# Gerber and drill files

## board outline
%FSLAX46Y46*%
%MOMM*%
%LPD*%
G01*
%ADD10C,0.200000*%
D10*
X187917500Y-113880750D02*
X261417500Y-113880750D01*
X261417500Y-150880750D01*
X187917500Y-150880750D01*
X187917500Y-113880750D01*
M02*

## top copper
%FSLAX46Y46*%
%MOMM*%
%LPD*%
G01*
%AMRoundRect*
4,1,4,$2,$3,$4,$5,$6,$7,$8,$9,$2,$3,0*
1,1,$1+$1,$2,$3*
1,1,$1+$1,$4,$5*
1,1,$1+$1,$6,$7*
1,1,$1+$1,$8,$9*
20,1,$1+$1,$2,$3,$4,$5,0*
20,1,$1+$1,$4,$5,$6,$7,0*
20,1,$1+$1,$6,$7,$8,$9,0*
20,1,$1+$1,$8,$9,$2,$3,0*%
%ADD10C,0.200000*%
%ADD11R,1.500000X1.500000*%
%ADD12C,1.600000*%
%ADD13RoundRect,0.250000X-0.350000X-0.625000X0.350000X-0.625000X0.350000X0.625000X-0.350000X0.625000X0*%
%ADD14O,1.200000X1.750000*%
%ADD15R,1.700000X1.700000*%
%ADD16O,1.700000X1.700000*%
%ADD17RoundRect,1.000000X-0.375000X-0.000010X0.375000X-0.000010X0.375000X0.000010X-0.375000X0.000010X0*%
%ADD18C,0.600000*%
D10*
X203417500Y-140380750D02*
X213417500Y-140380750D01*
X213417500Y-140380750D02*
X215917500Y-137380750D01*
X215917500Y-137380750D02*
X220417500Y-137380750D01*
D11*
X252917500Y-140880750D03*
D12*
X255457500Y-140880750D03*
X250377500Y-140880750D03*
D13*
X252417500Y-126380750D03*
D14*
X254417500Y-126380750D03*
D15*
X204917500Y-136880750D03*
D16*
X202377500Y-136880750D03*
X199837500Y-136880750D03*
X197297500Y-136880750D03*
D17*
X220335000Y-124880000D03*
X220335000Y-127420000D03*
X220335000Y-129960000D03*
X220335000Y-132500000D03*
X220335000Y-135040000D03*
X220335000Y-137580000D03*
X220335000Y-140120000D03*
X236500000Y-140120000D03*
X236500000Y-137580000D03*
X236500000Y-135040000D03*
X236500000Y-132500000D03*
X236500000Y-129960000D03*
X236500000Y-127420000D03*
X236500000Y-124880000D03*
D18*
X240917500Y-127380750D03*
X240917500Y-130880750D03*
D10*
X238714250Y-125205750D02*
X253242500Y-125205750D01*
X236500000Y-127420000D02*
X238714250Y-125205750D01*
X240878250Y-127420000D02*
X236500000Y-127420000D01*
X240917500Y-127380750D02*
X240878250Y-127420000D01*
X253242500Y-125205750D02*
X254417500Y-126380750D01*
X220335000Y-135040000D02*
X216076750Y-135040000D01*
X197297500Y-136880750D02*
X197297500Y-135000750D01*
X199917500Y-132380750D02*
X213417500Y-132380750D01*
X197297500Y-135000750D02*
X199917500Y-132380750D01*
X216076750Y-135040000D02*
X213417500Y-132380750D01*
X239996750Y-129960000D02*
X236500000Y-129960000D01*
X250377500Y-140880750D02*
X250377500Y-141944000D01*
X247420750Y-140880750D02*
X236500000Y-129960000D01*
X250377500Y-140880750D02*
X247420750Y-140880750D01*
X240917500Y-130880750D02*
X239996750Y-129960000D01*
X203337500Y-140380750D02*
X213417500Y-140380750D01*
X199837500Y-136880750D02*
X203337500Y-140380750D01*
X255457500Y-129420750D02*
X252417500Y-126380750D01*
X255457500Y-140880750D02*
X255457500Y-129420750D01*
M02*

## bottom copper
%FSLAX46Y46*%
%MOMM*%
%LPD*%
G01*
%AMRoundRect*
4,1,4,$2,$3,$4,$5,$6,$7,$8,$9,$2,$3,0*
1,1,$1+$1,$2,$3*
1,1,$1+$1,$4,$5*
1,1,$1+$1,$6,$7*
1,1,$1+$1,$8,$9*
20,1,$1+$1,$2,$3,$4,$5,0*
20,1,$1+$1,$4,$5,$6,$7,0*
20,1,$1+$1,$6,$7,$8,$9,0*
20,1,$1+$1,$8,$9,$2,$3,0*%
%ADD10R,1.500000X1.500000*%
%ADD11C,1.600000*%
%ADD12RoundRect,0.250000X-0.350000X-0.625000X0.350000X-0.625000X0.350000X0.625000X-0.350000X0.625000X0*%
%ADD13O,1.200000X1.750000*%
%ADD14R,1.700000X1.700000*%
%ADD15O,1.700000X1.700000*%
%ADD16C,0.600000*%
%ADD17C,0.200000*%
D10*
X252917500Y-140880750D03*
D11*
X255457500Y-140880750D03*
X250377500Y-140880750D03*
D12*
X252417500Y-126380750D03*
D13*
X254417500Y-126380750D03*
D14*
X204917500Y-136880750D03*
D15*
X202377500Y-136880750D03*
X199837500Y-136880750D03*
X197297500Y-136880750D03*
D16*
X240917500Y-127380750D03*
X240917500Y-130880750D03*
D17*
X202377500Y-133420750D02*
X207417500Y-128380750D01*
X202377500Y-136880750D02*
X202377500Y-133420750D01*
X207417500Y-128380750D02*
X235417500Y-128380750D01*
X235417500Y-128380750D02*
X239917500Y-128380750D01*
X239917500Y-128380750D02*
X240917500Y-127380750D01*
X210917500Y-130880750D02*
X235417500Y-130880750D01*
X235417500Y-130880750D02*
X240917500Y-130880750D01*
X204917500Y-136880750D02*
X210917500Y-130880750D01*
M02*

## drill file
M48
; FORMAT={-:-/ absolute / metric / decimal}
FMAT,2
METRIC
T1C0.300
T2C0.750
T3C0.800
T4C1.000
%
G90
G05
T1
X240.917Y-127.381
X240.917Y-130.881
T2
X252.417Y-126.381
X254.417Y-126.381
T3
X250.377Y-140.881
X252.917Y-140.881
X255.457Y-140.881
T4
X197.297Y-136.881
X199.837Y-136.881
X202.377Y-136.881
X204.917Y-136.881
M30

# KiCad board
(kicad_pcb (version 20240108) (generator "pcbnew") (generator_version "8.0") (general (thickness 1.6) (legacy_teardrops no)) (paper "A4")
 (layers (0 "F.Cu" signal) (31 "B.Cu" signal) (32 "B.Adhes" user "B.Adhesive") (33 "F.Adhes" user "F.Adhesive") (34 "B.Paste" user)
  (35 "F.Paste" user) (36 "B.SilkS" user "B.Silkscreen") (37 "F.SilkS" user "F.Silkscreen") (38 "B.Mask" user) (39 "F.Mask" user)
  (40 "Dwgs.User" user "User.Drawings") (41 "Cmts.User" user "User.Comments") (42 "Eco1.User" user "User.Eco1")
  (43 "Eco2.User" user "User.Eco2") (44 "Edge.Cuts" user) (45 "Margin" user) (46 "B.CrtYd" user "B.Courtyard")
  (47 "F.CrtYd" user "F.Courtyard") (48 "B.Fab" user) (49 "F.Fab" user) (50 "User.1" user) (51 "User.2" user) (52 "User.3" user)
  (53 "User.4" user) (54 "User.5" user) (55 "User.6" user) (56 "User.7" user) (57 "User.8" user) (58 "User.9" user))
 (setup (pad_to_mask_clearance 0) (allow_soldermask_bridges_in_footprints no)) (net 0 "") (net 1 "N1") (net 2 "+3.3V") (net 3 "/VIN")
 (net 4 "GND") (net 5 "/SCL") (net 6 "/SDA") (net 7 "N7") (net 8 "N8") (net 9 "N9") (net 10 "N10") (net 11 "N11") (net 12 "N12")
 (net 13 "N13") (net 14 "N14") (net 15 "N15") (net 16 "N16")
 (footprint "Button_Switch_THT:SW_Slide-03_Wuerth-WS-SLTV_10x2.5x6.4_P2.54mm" (layer "F.Cu") (at 252.9175 140.88075 180)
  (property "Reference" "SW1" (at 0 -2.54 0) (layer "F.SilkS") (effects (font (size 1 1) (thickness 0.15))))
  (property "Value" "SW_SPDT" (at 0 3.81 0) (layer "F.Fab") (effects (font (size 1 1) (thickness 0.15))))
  (pad "1" thru_hole rect (at 0 0 180) (size 1.5 1.5) (drill 0.8) (layers "*.Cu" "*.Mask") (remove_unused_layers no) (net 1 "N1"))
  (pad "2" thru_hole circle (at -2.54 0 180) (size 1.6 1.6) (drill 0.8) (layers "*.Cu" "*.Mask") (remove_unused_layers no) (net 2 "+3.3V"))
  (pad "3" thru_hole circle (at 2.54 0 180) (size 1.6 1.6) (drill 0.8) (layers "*.Cu" "*.Mask") (remove_unused_layers no) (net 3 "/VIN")))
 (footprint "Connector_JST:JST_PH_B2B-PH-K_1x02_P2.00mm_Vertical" (layer "F.Cu") (at 252.4175 126.38075)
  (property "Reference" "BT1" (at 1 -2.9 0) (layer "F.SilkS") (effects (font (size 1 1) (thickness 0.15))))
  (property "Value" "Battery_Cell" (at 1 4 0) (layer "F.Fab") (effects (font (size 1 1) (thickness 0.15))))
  (pad "1" thru_hole roundrect (at 0 0) (size 1.2 1.75) (drill 0.75) (layers "*.Cu" "*.Mask") (remove_unused_layers no)
   (roundrect_rratio 0.208333) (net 2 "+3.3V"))
  (pad "2" thru_hole oval (at 2 0) (size 1.2 1.75) (drill 0.75) (layers "*.Cu" "*.Mask") (remove_unused_layers no) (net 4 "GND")))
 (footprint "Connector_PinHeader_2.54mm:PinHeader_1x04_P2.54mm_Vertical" (layer "F.Cu") (at 204.9175 136.88075 -90)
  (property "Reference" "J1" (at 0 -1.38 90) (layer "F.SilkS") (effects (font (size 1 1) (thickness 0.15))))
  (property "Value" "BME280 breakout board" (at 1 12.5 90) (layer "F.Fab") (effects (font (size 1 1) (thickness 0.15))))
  (pad "1" thru_hole rect (at 0 0 270) (size 1.7 1.7) (drill 1) (layers "*.Cu" "*.Mask") (remove_unused_layers no) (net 3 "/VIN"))
  (pad "2" thru_hole oval (at 0 2.54 270) (size 1.7 1.7) (drill 1) (layers "*.Cu" "*.Mask") (remove_unused_layers no) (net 4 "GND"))
  (pad "3" thru_hole oval (at 0 5.08 270) (size 1.7 1.7) (drill 1) (layers "*.Cu" "*.Mask") (remove_unused_layers no) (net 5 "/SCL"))
  (pad "4" thru_hole oval (at 0 7.62 270) (size 1.7 1.7) (drill 1) (layers "*.Cu" "*.Mask") (remove_unused_layers no) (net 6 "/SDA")))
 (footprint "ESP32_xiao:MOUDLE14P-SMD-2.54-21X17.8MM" (layer "F.Cu") (at 219.5 143)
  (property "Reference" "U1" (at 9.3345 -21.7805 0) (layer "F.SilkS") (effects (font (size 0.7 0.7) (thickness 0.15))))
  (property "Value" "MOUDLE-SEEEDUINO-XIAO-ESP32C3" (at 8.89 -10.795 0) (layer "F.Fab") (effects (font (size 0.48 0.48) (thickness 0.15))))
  (pad "1" smd roundrect (at 0.835 -18.12) (size 2.75 2) (layers "F.Cu" "F.Paste" "F.Mask") (roundrect_rratio 0.5) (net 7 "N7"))
  (pad "2" smd roundrect (at 0.835 -15.58) (size 2.75 2) (layers "F.Cu" "F.Paste" "F.Mask") (roundrect_rratio 0.5) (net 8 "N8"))
  (pad "3" smd roundrect (at 0.835 -13.04) (size 2.75 2) (layers "F.Cu" "F.Paste" "F.Mask") (roundrect_rratio 0.5) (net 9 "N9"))
  (pad "4" smd roundrect (at 0.835 -10.5) (size 2.75 2) (layers "F.Cu" "F.Paste" "F.Mask") (roundrect_rratio 0.5) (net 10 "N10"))
  (pad "5" smd roundrect (at 0.835 -7.96) (size 2.75 2) (layers "F.Cu" "F.Paste" "F.Mask") (roundrect_rratio 0.5) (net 6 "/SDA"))
  (pad "6" smd roundrect (at 0.835 -5.42) (size 2.75 2) (layers "F.Cu" "F.Paste" "F.Mask") (roundrect_rratio 0.5) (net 5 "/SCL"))
  (pad "7" smd roundrect (at 0.835 -2.88) (size 2.75 2) (layers "F.Cu" "F.Paste" "F.Mask") (roundrect_rratio 0.5) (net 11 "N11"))
  (pad "8" smd roundrect (at 17 -2.88) (size 2.75 2) (layers "F.Cu" "F.Paste" "F.Mask") (roundrect_rratio 0.5) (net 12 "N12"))
  (pad "9" smd roundrect (at 17 -5.42) (size 2.75 2) (layers "F.Cu" "F.Paste" "F.Mask") (roundrect_rratio 0.5) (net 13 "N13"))
  (pad "10" smd roundrect (at 17 -7.96) (size 2.75 2) (layers "F.Cu" "F.Paste" "F.Mask") (roundrect_rratio 0.5) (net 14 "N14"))
  (pad "11" smd roundrect (at 17 -10.5) (size 2.75 2) (layers "F.Cu" "F.Paste" "F.Mask") (roundrect_rratio 0.5) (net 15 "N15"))
  (pad "12" smd roundrect (at 17 -13.04) (size 2.75 2) (layers "F.Cu" "F.Paste" "F.Mask") (roundrect_rratio 0.5) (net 3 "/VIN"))
  (pad "13" smd roundrect (at 17 -15.58) (size 2.75 2) (layers "F.Cu" "F.Paste" "F.Mask") (roundrect_rratio 0.5) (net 4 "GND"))
  (pad "14" smd roundrect (at 17 -18.12) (size 2.75 2) (layers "F.Cu" "F.Paste" "F.Mask") (roundrect_rratio 0.5) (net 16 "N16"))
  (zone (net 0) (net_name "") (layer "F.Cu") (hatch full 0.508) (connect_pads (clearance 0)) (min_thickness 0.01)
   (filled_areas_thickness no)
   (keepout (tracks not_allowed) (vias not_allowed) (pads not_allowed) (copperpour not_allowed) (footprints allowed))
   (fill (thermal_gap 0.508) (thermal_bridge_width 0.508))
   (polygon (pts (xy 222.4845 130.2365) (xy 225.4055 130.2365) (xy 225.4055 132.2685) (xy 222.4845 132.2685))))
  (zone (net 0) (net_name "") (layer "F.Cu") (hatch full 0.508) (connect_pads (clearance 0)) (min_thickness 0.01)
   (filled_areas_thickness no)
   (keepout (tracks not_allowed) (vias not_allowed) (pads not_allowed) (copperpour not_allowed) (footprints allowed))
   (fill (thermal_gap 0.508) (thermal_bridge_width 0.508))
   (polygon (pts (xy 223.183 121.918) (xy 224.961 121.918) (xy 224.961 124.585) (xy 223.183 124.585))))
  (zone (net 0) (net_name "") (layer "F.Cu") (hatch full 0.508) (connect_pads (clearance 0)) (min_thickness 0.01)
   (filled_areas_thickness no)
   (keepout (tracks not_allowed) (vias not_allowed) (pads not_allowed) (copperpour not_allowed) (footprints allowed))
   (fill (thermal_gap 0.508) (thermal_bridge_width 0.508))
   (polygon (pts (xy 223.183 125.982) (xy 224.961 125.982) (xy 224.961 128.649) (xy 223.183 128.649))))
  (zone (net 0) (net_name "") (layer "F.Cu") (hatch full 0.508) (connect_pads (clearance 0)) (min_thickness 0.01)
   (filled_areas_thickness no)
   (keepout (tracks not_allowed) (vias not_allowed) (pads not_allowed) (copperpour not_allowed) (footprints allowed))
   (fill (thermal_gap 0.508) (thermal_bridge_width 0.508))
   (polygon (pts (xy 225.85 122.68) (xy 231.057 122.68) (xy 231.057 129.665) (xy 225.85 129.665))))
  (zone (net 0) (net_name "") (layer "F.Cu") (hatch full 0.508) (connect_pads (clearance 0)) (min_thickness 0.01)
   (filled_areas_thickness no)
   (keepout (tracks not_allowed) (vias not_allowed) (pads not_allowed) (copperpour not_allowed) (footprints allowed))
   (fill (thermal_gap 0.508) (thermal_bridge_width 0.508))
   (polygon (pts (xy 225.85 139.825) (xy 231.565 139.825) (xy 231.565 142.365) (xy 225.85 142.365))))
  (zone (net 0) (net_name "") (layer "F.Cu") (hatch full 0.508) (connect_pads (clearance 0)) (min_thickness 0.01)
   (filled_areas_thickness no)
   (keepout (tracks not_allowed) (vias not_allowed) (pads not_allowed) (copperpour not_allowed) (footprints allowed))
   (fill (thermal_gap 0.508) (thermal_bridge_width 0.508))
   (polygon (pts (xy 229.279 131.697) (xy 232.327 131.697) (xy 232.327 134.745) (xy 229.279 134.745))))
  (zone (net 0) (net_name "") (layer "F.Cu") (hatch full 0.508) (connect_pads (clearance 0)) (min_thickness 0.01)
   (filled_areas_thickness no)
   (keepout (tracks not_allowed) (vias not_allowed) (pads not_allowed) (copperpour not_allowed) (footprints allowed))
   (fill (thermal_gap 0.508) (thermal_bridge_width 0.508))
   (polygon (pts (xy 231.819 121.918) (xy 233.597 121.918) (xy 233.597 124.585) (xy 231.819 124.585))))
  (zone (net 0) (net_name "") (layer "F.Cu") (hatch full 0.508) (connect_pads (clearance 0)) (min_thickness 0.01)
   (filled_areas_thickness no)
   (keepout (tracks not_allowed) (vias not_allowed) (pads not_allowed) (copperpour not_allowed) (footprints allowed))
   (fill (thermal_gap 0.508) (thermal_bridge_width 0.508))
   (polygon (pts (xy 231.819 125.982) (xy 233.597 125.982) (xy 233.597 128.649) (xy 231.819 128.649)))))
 (gr_line (start 203.4175 140.38075) (end 213.4175 140.38075) (stroke (width 0.2) (type default)) (layer "F.Cu") (net 5))
 (gr_line (start 213.4175 140.38075) (end 215.9175 137.38075) (stroke (width 0.2) (type default)) (layer "F.Cu") (net 5))
 (gr_line (start 215.9175 137.38075) (end 220.4175 137.38075) (stroke (width 0.2) (type default)) (layer "F.Cu") (net 5))
 (gr_rect (start 187.9175 113.88075) (end 261.4175 150.88075) (stroke (width 0.2) (type default)) (fill none) (layer "Edge.Cuts"))
 (segment (start 238.71425 125.20575) (end 253.2425 125.20575) (width 0.2) (layer "F.Cu") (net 4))
 (segment (start 236.5 127.42) (end 238.71425 125.20575) (width 0.2) (layer "F.Cu") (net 4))
 (segment (start 240.87825 127.42) (end 236.5 127.42) (width 0.2) (layer "F.Cu") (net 4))
 (segment (start 240.9175 127.38075) (end 240.87825 127.42) (width 0.2) (layer "F.Cu") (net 4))
 (segment (start 253.2425 125.20575) (end 254.4175 126.38075) (width 0.2) (layer "F.Cu") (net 4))
 (via (at 240.9175 127.38075) (size 0.6) (drill 0.3) (layers "F.Cu" "B.Cu") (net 4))
 (segment (start 202.3775 133.42075) (end 207.4175 128.38075) (width 0.2) (layer "B.Cu") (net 4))
 (segment (start 202.3775 136.88075) (end 202.3775 133.42075) (width 0.2) (layer "B.Cu") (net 4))
 (segment (start 207.4175 128.38075) (end 235.4175 128.38075) (width 0.2) (layer "B.Cu") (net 4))
 (segment (start 235.4175 128.38075) (end 239.9175 128.38075) (width 0.2) (layer "B.Cu") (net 4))
 (segment (start 239.9175 128.38075) (end 240.9175 127.38075) (width 0.2) (layer "B.Cu") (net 4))
 (segment (start 220.335 135.04) (end 216.07675 135.04) (width 0.2) (layer "F.Cu") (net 6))
 (segment (start 197.2975 136.88075) (end 197.2975 135.00075) (width 0.2) (layer "F.Cu") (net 6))
 (segment (start 199.9175 132.38075) (end 213.4175 132.38075) (width 0.2) (layer "F.Cu") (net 6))
 (segment (start 197.2975 135.00075) (end 199.9175 132.38075) (width 0.2) (layer "F.Cu") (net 6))
 (segment (start 216.07675 135.04) (end 213.4175 132.38075) (width 0.2) (layer "F.Cu") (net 6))
 (segment (start 239.99675 129.96) (end 236.5 129.96) (width 0.2) (layer "F.Cu") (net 3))
 (segment (start 250.3775 140.88075) (end 250.3775 141.944) (width 0.2) (layer "F.Cu") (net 3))
 (segment (start 247.42075 140.88075) (end 236.5 129.96) (width 0.2) (layer "F.Cu") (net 3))
 (segment (start 250.3775 140.88075) (end 247.42075 140.88075) (width 0.2) (layer "F.Cu") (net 3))
 (segment (start 240.9175 130.88075) (end 239.99675 129.96) (width 0.2) (layer "F.Cu") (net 3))
 (via (at 240.9175 130.88075) (size 0.6) (drill 0.3) (layers "F.Cu" "B.Cu") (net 3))
 (segment (start 210.9175 130.88075) (end 235.4175 130.88075) (width 0.2) (layer "B.Cu") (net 3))
 (segment (start 235.4175 130.88075) (end 240.9175 130.88075) (width 0.2) (layer "B.Cu") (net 3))
 (segment (start 204.9175 136.88075) (end 210.9175 130.88075) (width 0.2) (layer "B.Cu") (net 3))
 (segment (start 203.3375 140.38075) (end 213.4175 140.38075) (width 0.2) (layer "F.Cu") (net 5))
 (segment (start 199.8375 136.88075) (end 203.3375 140.38075) (width 0.2) (layer "F.Cu") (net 5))
 (segment (start 255.4575 129.42075) (end 252.4175 126.38075) (width 0.2) (layer "F.Cu") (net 2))
 (segment (start 255.4575 140.88075) (end 255.4575 129.42075) (width 0.2) (layer "F.Cu") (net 2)))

